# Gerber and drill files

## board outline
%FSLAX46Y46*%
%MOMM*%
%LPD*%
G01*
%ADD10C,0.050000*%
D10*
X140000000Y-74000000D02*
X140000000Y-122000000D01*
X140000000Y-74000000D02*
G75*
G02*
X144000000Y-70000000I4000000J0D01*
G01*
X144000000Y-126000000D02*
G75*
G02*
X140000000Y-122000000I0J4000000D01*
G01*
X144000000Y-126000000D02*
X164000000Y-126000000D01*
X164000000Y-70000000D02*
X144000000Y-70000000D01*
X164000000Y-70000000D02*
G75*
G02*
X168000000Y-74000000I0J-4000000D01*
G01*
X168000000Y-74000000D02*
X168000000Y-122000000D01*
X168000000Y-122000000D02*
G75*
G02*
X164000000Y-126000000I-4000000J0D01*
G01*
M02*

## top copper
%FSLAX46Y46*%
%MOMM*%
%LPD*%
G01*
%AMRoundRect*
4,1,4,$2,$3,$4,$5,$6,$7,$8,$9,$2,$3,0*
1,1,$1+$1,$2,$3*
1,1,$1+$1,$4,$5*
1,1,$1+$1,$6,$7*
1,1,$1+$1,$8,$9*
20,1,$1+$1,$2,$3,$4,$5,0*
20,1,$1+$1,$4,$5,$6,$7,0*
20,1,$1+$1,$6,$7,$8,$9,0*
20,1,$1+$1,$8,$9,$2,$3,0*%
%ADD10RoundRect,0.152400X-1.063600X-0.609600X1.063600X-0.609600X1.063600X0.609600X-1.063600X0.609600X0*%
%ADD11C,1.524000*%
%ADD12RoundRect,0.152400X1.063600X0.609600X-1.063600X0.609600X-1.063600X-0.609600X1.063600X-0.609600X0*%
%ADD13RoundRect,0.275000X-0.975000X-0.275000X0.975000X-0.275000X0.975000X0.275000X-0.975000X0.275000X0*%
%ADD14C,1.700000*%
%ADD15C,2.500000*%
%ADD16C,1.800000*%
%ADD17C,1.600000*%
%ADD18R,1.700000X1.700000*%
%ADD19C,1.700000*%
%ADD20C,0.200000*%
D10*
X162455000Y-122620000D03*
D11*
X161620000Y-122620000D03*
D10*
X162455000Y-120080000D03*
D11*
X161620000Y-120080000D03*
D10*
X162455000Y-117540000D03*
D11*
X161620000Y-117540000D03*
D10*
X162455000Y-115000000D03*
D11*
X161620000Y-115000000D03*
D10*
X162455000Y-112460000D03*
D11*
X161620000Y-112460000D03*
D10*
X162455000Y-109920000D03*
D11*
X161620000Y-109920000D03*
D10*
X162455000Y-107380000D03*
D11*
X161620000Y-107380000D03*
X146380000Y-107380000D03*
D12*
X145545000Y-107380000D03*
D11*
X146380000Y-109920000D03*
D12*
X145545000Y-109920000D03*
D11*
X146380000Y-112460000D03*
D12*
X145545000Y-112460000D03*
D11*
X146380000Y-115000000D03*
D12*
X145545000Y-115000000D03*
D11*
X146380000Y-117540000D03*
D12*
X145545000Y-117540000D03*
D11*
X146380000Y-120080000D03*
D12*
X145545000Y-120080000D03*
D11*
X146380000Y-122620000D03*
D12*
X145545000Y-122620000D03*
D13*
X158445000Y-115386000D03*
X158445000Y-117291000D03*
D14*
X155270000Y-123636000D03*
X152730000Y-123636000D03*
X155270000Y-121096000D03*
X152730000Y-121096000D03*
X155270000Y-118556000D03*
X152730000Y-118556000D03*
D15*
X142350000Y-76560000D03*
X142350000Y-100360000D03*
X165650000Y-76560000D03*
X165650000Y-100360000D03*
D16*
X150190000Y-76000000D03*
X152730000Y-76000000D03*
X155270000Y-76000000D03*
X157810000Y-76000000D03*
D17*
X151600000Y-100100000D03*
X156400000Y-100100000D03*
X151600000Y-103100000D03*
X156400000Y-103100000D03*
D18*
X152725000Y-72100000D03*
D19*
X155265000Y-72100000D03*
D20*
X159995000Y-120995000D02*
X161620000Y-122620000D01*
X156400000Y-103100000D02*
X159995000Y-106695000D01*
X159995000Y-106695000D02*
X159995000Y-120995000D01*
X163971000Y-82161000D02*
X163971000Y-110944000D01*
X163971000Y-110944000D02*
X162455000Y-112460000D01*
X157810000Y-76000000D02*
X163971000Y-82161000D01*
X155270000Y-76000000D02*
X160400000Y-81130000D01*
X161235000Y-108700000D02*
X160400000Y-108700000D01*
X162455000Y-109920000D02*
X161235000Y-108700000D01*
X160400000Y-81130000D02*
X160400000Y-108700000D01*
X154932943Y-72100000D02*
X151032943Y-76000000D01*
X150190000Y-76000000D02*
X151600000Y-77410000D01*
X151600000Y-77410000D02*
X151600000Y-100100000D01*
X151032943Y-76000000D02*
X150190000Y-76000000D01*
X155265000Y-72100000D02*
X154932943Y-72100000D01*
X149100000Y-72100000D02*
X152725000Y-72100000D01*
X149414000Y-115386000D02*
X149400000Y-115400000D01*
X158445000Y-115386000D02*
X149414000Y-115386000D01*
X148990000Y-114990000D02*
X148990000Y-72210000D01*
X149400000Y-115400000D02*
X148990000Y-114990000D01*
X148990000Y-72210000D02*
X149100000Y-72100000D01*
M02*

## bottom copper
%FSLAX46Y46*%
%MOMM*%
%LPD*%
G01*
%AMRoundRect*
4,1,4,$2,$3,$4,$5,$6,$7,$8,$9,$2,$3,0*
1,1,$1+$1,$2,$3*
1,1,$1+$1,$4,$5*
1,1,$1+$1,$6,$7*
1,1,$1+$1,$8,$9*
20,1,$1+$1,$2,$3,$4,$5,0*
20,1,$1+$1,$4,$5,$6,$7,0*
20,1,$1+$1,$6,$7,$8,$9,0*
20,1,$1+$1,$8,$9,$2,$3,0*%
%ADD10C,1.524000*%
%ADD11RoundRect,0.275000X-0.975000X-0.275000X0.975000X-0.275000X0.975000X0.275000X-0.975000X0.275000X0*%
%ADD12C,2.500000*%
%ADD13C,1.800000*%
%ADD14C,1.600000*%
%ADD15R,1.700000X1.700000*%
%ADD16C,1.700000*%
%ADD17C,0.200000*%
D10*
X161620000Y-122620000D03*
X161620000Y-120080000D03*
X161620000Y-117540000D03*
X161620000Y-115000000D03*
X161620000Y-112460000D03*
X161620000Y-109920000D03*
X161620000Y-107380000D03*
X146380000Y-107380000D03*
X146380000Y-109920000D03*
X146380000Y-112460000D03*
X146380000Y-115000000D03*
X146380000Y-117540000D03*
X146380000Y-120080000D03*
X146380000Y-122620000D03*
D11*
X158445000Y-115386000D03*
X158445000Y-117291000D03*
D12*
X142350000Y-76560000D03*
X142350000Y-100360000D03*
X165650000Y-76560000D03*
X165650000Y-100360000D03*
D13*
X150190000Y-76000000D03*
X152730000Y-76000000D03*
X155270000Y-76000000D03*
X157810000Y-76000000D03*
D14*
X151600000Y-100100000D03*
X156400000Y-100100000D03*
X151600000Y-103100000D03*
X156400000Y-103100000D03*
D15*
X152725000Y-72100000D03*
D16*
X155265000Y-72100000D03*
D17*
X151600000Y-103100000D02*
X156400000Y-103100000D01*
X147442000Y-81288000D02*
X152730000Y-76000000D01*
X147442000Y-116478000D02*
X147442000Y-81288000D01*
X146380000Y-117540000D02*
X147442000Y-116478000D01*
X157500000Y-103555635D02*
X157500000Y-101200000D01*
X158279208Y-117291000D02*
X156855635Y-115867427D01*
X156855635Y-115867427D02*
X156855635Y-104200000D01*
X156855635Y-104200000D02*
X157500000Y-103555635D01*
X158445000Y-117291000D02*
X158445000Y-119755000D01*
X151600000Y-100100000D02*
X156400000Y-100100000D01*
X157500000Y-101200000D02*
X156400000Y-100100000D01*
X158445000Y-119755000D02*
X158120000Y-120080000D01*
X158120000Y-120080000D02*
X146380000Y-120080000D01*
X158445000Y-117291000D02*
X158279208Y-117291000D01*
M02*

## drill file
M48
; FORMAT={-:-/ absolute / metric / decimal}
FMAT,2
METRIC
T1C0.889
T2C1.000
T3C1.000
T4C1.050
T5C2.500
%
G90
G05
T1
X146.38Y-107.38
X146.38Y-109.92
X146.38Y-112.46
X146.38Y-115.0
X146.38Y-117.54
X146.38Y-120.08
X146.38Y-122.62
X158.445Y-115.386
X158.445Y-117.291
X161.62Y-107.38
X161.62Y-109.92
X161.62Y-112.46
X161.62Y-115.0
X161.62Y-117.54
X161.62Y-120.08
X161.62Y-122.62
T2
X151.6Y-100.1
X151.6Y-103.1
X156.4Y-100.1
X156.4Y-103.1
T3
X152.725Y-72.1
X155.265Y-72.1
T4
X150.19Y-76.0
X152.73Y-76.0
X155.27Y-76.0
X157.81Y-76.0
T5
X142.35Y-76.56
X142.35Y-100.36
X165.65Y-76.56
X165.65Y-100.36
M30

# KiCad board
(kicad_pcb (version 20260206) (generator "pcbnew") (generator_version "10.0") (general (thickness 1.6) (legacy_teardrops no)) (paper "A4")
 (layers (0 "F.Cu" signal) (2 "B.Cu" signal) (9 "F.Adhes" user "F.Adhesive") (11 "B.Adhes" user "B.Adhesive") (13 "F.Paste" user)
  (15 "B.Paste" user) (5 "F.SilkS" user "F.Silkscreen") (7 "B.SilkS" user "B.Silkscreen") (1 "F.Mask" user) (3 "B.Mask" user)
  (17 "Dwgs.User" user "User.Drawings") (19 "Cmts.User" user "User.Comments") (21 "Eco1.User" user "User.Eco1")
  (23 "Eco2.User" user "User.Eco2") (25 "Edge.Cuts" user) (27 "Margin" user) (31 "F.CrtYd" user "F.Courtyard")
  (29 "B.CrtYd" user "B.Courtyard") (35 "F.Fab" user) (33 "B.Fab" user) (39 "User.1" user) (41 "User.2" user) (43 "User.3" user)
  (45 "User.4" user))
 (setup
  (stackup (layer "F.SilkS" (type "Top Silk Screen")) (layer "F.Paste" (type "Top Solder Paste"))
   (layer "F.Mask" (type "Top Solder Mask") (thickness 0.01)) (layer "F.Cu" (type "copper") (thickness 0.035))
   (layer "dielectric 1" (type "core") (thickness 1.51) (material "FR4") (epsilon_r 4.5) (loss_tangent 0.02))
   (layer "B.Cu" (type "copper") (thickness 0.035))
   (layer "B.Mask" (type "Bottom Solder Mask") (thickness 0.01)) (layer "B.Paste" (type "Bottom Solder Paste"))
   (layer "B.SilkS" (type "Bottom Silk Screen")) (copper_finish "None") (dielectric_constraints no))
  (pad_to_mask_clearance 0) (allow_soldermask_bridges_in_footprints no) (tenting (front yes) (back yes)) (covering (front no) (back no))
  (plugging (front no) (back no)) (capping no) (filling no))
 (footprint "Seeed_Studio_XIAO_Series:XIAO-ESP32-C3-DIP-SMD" (layer "F.Cu") (at 154 115 -90)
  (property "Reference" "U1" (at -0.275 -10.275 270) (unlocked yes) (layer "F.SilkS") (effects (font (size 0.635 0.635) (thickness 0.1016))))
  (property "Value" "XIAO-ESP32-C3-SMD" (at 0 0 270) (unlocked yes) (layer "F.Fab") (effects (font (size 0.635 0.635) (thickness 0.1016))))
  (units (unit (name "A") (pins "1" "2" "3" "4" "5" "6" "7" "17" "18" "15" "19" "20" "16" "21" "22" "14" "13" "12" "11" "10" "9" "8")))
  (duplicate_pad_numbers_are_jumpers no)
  (pad "1" smd roundrect (at 7.62 -8.455) (size 2.432 1.524) (layers "F.Cu" "F.Mask") (roundrect_rratio 0.1) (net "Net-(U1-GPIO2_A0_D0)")
   (thermal_bridge_angle 45))
  (pad "1" thru_hole circle (at 7.62 -7.62) (size 1.524 1.524) (drill 0.889) (layers "*.Cu" "*.Mask") (remove_unused_layers no)
   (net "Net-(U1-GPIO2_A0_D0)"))
  (pad "2" smd roundrect (at 5.08 -8.455) (size 2.432 1.524) (layers "F.Cu" "F.Mask") (roundrect_rratio 0.1)
   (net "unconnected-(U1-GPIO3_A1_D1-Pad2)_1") (thermal_bridge_angle 45))
  (pad "2" thru_hole circle (at 5.08 -7.62) (size 1.524 1.524) (drill 0.889) (layers "*.Cu" "*.Mask") (remove_unused_layers no)
   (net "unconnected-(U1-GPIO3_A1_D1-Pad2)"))
  (pad "3" smd roundrect (at 2.54 -8.455) (size 2.432 1.524) (layers "F.Cu" "F.Mask") (roundrect_rratio 0.1)
   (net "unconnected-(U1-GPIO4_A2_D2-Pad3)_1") (thermal_bridge_angle 45))
  (pad "3" thru_hole circle (at 2.54 -7.62) (size 1.524 1.524) (drill 0.889) (layers "*.Cu" "*.Mask") (remove_unused_layers no)
   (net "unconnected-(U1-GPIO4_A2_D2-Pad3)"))
  (pad "4" smd roundrect (at 0 -8.455) (size 2.432 1.524) (layers "F.Cu" "F.Mask") (roundrect_rratio 0.1)
   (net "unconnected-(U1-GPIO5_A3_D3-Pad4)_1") (thermal_bridge_angle 45))
  (pad "4" thru_hole circle (at 0 -7.62) (size 1.524 1.524) (drill 0.889) (layers "*.Cu" "*.Mask") (remove_unused_layers no)
   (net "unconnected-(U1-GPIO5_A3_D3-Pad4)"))
  (pad "5" smd roundrect (at -2.54 -8.455) (size 2.432 1.524) (layers "F.Cu" "F.Mask") (roundrect_rratio 0.1) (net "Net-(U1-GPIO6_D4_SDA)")
   (thermal_bridge_angle 45))
  (pad "5" thru_hole circle (at -2.54 -7.62) (size 1.524 1.524) (drill 0.889) (layers "*.Cu" "*.Mask") (remove_unused_layers no)
   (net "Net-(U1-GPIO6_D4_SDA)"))
  (pad "6" smd roundrect (at -5.08 -8.455) (size 2.432 1.524) (layers "F.Cu" "F.Mask") (roundrect_rratio 0.1) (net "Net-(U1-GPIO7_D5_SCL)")
   (thermal_bridge_angle 45))
  (pad "6" thru_hole circle (at -5.08 -7.62) (size 1.524 1.524) (drill 0.889) (layers "*.Cu" "*.Mask") (remove_unused_layers no)
   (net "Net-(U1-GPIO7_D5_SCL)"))
  (pad "7" smd roundrect (at -7.62 -8.455) (size 2.432 1.524) (layers "F.Cu" "F.Mask") (roundrect_rratio 0.1)
   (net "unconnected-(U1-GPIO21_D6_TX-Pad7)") (thermal_bridge_angle 45))
  (pad "7" thru_hole circle (at -7.62 -7.62) (size 1.524 1.524) (drill 0.889) (layers "*.Cu" "*.Mask") (remove_unused_layers no)
   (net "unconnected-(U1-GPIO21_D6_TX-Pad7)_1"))
  (pad "8" thru_hole circle (at -7.62 7.62 180) (size 1.524 1.524) (drill 0.889) (layers "*.Cu" "*.Mask") (remove_unused_layers no)
   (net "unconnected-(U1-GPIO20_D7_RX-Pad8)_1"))
  (pad "8" smd roundrect (at -7.62 8.455 180) (size 2.432 1.524) (layers "F.Cu" "F.Mask") (roundrect_rratio 0.1)
   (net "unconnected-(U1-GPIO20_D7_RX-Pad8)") (thermal_bridge_angle 45))
  (pad "9" thru_hole circle (at -5.08 7.62 180) (size 1.524 1.524) (drill 0.889) (layers "*.Cu" "*.Mask") (remove_unused_layers no)
   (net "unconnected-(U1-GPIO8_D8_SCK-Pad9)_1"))
  (pad "9" smd roundrect (at -5.08 8.455 180) (size 2.432 1.524) (layers "F.Cu" "F.Mask") (roundrect_rratio 0.1)
   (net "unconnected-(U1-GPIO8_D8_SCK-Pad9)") (thermal_bridge_angle 45))
  (pad "10" thru_hole circle (at -2.54 7.62 180) (size 1.524 1.524) (drill 0.889) (layers "*.Cu" "*.Mask") (remove_unused_layers no)
   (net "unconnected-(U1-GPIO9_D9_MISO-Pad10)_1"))
  (pad "10" smd roundrect (at -2.54 8.455 180) (size 2.432 1.524) (layers "F.Cu" "F.Mask") (roundrect_rratio 0.1)
   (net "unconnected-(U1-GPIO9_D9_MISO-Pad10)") (thermal_bridge_angle 45))
  (pad "11" thru_hole circle (at 0 7.62 180) (size 1.524 1.524) (drill 0.889) (layers "*.Cu" "*.Mask") (remove_unused_layers no)
   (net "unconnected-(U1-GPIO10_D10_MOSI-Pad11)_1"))
  (pad "11" smd roundrect (at 0 8.455 180) (size 2.432 1.524) (layers "F.Cu" "F.Mask") (roundrect_rratio 0.1)
   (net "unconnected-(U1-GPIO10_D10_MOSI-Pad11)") (thermal_bridge_angle 45))
  (pad "12" thru_hole circle (at 2.54 7.62 180) (size 1.524 1.524) (drill 0.889) (layers "*.Cu" "*.Mask") (remove_unused_layers no)
   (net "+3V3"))
  (pad "12" smd roundrect (at 2.54 8.455 180) (size 2.432 1.524) (layers "F.Cu" "F.Mask") (roundrect_rratio 0.1) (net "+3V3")
   (thermal_bridge_angle 45))
  (pad "13" thru_hole circle (at 5.08 7.62 180) (size 1.524 1.524) (drill 0.889) (layers "*.Cu" "*.Mask") (remove_unused_layers no)
   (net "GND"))
  (pad "13" smd roundrect (at 5.08 8.455 180) (size 2.432 1.524) (layers "F.Cu" "F.Mask") (roundrect_rratio 0.1) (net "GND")
   (thermal_bridge_angle 45))
  (pad "14" thru_hole circle (at 7.62 7.62 180) (size 1.524 1.524) (drill 0.889) (layers "*.Cu" "*.Mask") (remove_unused_layers no)
   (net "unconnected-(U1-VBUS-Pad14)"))
  (pad "14" smd roundrect (at 7.62 8.455 180) (size 2.432 1.524) (layers "F.Cu" "F.Mask") (roundrect_rratio 0.1)
   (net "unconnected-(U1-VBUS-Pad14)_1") (thermal_bridge_angle 45))
  (pad "15" thru_hole roundrect (at 0.386 -4.445) (size 2.5 1.1) (drill 0.889) (layers "*.Cu" "*.Mask") (remove_unused_layers no)
   (roundrect_rratio 0.25) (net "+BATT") (thermal_bridge_angle 45))
  (pad "16" thru_hole roundrect (at 2.291 -4.445) (size 2.5 1.1) (drill 0.889) (layers "*.Cu" "*.Mask") (remove_unused_layers no)
   (roundrect_rratio 0.25) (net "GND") (thermal_bridge_angle 45))
  (pad "17" smd circle (at 8.636 -1.27 180) (size 1.7 1.7) (layers "F.Cu" "F.Mask" "F.Paste") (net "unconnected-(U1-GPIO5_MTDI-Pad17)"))
  (pad "18" smd circle (at 8.636 1.27 180) (size 1.7 1.7) (layers "F.Cu" "F.Mask" "F.Paste") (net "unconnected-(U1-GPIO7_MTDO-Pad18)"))
  (pad "19" smd circle (at 6.096 -1.27 180) (size 1.7 1.7) (layers "F.Cu" "F.Mask" "F.Paste") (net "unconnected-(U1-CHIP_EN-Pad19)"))
  (pad "20" smd circle (at 6.096 1.27 180) (size 1.7 1.7) (layers "F.Cu" "F.Mask" "F.Paste") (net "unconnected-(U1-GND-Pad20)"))
  (pad "21" smd circle (at 3.556 -1.27 180) (size 1.7 1.7) (layers "F.Cu" "F.Mask" "F.Paste") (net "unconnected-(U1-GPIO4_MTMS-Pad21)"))
  (pad "22" smd circle (at 3.556 1.27 180) (size 1.7 1.7) (layers "F.Cu" "F.Mask" "F.Paste") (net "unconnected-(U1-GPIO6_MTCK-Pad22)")))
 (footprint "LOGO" (layer "F.Cu") (at 161.684622 76.284609)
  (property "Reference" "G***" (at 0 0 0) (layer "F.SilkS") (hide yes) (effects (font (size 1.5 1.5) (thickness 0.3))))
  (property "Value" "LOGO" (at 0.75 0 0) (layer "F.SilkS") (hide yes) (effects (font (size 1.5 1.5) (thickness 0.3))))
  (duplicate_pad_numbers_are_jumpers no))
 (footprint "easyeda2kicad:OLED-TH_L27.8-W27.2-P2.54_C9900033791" (layer "F.Cu") (at 154 76)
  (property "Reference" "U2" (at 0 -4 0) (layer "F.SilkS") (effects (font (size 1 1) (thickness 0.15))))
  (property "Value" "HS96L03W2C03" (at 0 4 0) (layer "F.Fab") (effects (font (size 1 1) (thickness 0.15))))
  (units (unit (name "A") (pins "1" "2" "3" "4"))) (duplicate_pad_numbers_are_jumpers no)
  (pad "" thru_hole circle (at -11.65 0.56) (size 2.5 2.5) (drill 2.5) (layers "*.Cu" "*.Mask") (remove_unused_layers no))
  (pad "" thru_hole circle (at -11.65 24.36) (size 2.5 2.5) (drill 2.5) (layers "*.Cu" "*.Mask") (remove_unused_layers no))
  (pad "" thru_hole circle (at 11.65 0.56) (size 2.5 2.5) (drill 2.5) (layers "*.Cu" "*.Mask") (remove_unused_layers no))
  (pad "" thru_hole circle (at 11.65 24.36) (size 2.5 2.5) (drill 2.5) (layers "*.Cu" "*.Mask") (remove_unused_layers no))
  (pad "1" thru_hole circle (at -3.81 0) (size 1.8 1.8) (drill 1.049986) (layers "*.Cu" "*.Mask") (remove_unused_layers no) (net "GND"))
  (pad "2" thru_hole circle (at -1.27 0) (size 1.8 1.8) (drill 1.049986) (layers "*.Cu" "*.Mask") (remove_unused_layers no) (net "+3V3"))
  (pad "3" thru_hole circle (at 1.27 0) (size 1.8 1.8) (drill 1.049986) (layers "*.Cu" "*.Mask") (remove_unused_layers no)
   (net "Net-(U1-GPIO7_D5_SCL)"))
  (pad "4" thru_hole circle (at 3.81 0) (size 1.8 1.8) (drill 1.049986) (layers "*.Cu" "*.Mask") (remove_unused_layers no)
   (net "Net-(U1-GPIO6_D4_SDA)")))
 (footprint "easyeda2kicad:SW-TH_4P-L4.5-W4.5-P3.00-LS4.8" (layer "F.Cu") (at 154 101.6)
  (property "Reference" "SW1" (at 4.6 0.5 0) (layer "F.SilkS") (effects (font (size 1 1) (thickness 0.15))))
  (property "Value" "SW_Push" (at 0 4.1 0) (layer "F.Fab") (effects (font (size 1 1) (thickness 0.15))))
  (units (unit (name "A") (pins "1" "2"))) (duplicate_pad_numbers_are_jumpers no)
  (pad "1" thru_hole circle (at -2.4 -1.5) (size 1.6 1.6) (drill 0.999998) (layers "*.Cu" "*.Mask") (remove_unused_layers no) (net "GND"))
  (pad "1" thru_hole circle (at 2.4 -1.5) (size 1.6 1.6) (drill 0.999998) (layers "*.Cu" "*.Mask") (remove_unused_layers no) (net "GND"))
  (pad "2" thru_hole circle (at -2.4 1.5) (size 1.6 1.6) (drill 0.999998) (layers "*.Cu" "*.Mask") (remove_unused_layers no)
   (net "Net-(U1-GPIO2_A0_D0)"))
  (pad "2" thru_hole circle (at 2.4 1.5) (size 1.6 1.6) (drill 0.999998) (layers "*.Cu" "*.Mask") (remove_unused_layers no)
   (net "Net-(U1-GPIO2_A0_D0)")))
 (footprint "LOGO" (layer "F.Cu") (at 144.1 104)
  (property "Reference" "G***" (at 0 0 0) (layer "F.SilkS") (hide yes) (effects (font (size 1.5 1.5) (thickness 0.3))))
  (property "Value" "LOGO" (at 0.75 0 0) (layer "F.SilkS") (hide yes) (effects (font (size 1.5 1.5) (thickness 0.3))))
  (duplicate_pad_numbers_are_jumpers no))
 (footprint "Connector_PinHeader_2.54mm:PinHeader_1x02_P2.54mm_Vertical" (layer "F.Cu") (at 152.725 72.1 90)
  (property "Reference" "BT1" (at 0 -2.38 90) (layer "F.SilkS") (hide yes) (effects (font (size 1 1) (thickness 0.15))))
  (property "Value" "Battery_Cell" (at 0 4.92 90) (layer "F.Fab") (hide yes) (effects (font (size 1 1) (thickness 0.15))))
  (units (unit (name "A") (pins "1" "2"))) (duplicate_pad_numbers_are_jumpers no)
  (pad "1" thru_hole rect (at 0 0 90) (size 1.7 1.7) (drill 1) (layers "*.Cu" "*.Mask") (remove_unused_layers no) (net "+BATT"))
  (pad "2" thru_hole circle (at 0 2.54 90) (size 1.7 1.7) (drill 1) (layers "*.Cu" "*.Mask") (remove_unused_layers no) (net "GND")))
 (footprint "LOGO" (layer "F.Cu") (at 146.4 76.1)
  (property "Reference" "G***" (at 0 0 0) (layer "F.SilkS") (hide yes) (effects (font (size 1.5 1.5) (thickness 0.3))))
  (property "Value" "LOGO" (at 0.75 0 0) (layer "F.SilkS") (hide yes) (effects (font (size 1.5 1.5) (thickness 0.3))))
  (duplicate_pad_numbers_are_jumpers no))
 (gr_line (start 140 74) (end 140 122) (stroke (width 0.05) (type default)) (layer "Edge.Cuts"))
 (gr_arc (start 140 74) (mid 141.171573 71.171573) (end 144 70) (stroke (width 0.05) (type default)) (layer "Edge.Cuts"))
 (gr_arc (start 144 126) (mid 141.171573 124.828427) (end 140 122) (stroke (width 0.05) (type default)) (layer "Edge.Cuts"))
 (gr_line (start 144 126) (end 164 126) (stroke (width 0.05) (type default)) (layer "Edge.Cuts"))
 (gr_line (start 164 70) (end 144 70) (stroke (width 0.05) (type default)) (layer "Edge.Cuts"))
 (gr_arc (start 164 70) (mid 166.828427 71.171573) (end 168 74) (stroke (width 0.05) (type default)) (layer "Edge.Cuts"))
 (gr_line (start 168 74) (end 168 122) (stroke (width 0.05) (type default)) (layer "Edge.Cuts"))
 (gr_arc (start 168 122) (mid 166.828427 124.828427) (end 164 126) (stroke (width 0.05) (type default)) (layer "Edge.Cuts"))
 (segment (start 159.995 120.995) (end 161.62 122.62) (width 0.2) (layer "F.Cu") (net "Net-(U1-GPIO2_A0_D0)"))
 (segment (start 156.4 103.1) (end 159.995 106.695) (width 0.2) (layer "F.Cu") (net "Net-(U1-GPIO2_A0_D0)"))
 (segment (start 159.995 106.695) (end 159.995 120.995) (width 0.2) (layer "F.Cu") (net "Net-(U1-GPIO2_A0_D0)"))
 (segment (start 151.6 103.1) (end 156.4 103.1) (width 0.2) (layer "B.Cu") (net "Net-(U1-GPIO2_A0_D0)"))
 (segment (start 163.971 82.161) (end 163.971 110.944) (width 0.2) (layer "F.Cu") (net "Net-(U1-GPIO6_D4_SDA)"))
 (segment (start 163.971 110.944) (end 162.455 112.46) (width 0.2) (layer "F.Cu") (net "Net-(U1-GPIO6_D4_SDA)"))
 (segment (start 157.81 76) (end 163.971 82.161) (width 0.2) (layer "F.Cu") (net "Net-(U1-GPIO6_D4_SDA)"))
 (segment (start 155.27 76) (end 160.4 81.13) (width 0.2) (layer "F.Cu") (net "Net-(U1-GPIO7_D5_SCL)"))
 (segment (start 161.235 108.7) (end 160.4 108.7) (width 0.2) (layer "F.Cu") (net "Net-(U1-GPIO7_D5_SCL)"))
 (segment (start 162.455 109.92) (end 161.235 108.7) (width 0.2) (layer "F.Cu") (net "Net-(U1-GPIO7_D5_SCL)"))
 (segment (start 160.4 81.13) (end 160.4 108.7) (width 0.2) (layer "F.Cu") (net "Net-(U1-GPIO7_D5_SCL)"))
 (segment (start 147.442 81.288) (end 152.73 76) (width 0.2) (layer "B.Cu") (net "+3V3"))
 (segment (start 147.442 116.478) (end 147.442 81.288) (width 0.2) (layer "B.Cu") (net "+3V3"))
 (segment (start 146.38 117.54) (end 147.442 116.478) (width 0.2) (layer "B.Cu") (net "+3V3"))
 (segment (start 154.932943 72.1) (end 151.032943 76) (width 0.2) (layer "F.Cu") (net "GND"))
 (segment (start 150.19 76) (end 151.6 77.41) (width 0.2) (layer "F.Cu") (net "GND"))
 (segment (start 151.6 77.41) (end 151.6 100.1) (width 0.2) (layer "F.Cu") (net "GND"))
 (segment (start 151.032943 76) (end 150.19 76) (width 0.2) (layer "F.Cu") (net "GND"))
 (segment (start 155.265 72.1) (end 154.932943 72.1) (width 0.2) (layer "F.Cu") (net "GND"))
 (segment (start 157.5 103.555635) (end 157.5 101.2) (width 0.2) (layer "B.Cu") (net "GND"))
 (segment (start 158.279208 117.291) (end 156.855635 115.867427) (width 0.2) (layer "B.Cu") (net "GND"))
 (segment (start 156.855635 115.867427) (end 156.855635 104.2) (width 0.2) (layer "B.Cu") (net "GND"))
 (segment (start 156.855635 104.2) (end 157.5 103.555635) (width 0.2) (layer "B.Cu") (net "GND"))
 (segment (start 158.445 117.291) (end 158.445 119.755) (width 0.2) (layer "B.Cu") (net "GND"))
 (segment (start 151.6 100.1) (end 156.4 100.1) (width 0.2) (layer "B.Cu") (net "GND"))
 (segment (start 157.5 101.2) (end 156.4 100.1) (width 0.2) (layer "B.Cu") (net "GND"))
 (segment (start 158.445 119.755) (end 158.12 120.08) (width 0.2) (layer "B.Cu") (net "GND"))
 (segment (start 158.12 120.08) (end 146.38 120.08) (width 0.2) (layer "B.Cu") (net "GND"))
 (segment (start 158.445 117.291) (end 158.279208 117.291) (width 0.2) (layer "B.Cu") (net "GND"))
 (segment (start 149.1 72.1) (end 152.725 72.1) (width 0.2) (layer "F.Cu") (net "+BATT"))
 (segment (start 149.414 115.386) (end 149.4 115.4) (width 0.2) (layer "F.Cu") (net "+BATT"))
 (segment (start 158.445 115.386) (end 149.414 115.386) (width 0.2) (layer "F.Cu") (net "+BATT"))
 (segment (start 148.99 114.99) (end 148.99 72.21) (width 0.2) (layer "F.Cu") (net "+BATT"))
 (segment (start 149.4 115.4) (end 148.99 114.99) (width 0.2) (layer "F.Cu") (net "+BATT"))
 (segment (start 148.99 72.21) (end 149.1 72.1) (width 0.2) (layer "F.Cu") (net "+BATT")))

